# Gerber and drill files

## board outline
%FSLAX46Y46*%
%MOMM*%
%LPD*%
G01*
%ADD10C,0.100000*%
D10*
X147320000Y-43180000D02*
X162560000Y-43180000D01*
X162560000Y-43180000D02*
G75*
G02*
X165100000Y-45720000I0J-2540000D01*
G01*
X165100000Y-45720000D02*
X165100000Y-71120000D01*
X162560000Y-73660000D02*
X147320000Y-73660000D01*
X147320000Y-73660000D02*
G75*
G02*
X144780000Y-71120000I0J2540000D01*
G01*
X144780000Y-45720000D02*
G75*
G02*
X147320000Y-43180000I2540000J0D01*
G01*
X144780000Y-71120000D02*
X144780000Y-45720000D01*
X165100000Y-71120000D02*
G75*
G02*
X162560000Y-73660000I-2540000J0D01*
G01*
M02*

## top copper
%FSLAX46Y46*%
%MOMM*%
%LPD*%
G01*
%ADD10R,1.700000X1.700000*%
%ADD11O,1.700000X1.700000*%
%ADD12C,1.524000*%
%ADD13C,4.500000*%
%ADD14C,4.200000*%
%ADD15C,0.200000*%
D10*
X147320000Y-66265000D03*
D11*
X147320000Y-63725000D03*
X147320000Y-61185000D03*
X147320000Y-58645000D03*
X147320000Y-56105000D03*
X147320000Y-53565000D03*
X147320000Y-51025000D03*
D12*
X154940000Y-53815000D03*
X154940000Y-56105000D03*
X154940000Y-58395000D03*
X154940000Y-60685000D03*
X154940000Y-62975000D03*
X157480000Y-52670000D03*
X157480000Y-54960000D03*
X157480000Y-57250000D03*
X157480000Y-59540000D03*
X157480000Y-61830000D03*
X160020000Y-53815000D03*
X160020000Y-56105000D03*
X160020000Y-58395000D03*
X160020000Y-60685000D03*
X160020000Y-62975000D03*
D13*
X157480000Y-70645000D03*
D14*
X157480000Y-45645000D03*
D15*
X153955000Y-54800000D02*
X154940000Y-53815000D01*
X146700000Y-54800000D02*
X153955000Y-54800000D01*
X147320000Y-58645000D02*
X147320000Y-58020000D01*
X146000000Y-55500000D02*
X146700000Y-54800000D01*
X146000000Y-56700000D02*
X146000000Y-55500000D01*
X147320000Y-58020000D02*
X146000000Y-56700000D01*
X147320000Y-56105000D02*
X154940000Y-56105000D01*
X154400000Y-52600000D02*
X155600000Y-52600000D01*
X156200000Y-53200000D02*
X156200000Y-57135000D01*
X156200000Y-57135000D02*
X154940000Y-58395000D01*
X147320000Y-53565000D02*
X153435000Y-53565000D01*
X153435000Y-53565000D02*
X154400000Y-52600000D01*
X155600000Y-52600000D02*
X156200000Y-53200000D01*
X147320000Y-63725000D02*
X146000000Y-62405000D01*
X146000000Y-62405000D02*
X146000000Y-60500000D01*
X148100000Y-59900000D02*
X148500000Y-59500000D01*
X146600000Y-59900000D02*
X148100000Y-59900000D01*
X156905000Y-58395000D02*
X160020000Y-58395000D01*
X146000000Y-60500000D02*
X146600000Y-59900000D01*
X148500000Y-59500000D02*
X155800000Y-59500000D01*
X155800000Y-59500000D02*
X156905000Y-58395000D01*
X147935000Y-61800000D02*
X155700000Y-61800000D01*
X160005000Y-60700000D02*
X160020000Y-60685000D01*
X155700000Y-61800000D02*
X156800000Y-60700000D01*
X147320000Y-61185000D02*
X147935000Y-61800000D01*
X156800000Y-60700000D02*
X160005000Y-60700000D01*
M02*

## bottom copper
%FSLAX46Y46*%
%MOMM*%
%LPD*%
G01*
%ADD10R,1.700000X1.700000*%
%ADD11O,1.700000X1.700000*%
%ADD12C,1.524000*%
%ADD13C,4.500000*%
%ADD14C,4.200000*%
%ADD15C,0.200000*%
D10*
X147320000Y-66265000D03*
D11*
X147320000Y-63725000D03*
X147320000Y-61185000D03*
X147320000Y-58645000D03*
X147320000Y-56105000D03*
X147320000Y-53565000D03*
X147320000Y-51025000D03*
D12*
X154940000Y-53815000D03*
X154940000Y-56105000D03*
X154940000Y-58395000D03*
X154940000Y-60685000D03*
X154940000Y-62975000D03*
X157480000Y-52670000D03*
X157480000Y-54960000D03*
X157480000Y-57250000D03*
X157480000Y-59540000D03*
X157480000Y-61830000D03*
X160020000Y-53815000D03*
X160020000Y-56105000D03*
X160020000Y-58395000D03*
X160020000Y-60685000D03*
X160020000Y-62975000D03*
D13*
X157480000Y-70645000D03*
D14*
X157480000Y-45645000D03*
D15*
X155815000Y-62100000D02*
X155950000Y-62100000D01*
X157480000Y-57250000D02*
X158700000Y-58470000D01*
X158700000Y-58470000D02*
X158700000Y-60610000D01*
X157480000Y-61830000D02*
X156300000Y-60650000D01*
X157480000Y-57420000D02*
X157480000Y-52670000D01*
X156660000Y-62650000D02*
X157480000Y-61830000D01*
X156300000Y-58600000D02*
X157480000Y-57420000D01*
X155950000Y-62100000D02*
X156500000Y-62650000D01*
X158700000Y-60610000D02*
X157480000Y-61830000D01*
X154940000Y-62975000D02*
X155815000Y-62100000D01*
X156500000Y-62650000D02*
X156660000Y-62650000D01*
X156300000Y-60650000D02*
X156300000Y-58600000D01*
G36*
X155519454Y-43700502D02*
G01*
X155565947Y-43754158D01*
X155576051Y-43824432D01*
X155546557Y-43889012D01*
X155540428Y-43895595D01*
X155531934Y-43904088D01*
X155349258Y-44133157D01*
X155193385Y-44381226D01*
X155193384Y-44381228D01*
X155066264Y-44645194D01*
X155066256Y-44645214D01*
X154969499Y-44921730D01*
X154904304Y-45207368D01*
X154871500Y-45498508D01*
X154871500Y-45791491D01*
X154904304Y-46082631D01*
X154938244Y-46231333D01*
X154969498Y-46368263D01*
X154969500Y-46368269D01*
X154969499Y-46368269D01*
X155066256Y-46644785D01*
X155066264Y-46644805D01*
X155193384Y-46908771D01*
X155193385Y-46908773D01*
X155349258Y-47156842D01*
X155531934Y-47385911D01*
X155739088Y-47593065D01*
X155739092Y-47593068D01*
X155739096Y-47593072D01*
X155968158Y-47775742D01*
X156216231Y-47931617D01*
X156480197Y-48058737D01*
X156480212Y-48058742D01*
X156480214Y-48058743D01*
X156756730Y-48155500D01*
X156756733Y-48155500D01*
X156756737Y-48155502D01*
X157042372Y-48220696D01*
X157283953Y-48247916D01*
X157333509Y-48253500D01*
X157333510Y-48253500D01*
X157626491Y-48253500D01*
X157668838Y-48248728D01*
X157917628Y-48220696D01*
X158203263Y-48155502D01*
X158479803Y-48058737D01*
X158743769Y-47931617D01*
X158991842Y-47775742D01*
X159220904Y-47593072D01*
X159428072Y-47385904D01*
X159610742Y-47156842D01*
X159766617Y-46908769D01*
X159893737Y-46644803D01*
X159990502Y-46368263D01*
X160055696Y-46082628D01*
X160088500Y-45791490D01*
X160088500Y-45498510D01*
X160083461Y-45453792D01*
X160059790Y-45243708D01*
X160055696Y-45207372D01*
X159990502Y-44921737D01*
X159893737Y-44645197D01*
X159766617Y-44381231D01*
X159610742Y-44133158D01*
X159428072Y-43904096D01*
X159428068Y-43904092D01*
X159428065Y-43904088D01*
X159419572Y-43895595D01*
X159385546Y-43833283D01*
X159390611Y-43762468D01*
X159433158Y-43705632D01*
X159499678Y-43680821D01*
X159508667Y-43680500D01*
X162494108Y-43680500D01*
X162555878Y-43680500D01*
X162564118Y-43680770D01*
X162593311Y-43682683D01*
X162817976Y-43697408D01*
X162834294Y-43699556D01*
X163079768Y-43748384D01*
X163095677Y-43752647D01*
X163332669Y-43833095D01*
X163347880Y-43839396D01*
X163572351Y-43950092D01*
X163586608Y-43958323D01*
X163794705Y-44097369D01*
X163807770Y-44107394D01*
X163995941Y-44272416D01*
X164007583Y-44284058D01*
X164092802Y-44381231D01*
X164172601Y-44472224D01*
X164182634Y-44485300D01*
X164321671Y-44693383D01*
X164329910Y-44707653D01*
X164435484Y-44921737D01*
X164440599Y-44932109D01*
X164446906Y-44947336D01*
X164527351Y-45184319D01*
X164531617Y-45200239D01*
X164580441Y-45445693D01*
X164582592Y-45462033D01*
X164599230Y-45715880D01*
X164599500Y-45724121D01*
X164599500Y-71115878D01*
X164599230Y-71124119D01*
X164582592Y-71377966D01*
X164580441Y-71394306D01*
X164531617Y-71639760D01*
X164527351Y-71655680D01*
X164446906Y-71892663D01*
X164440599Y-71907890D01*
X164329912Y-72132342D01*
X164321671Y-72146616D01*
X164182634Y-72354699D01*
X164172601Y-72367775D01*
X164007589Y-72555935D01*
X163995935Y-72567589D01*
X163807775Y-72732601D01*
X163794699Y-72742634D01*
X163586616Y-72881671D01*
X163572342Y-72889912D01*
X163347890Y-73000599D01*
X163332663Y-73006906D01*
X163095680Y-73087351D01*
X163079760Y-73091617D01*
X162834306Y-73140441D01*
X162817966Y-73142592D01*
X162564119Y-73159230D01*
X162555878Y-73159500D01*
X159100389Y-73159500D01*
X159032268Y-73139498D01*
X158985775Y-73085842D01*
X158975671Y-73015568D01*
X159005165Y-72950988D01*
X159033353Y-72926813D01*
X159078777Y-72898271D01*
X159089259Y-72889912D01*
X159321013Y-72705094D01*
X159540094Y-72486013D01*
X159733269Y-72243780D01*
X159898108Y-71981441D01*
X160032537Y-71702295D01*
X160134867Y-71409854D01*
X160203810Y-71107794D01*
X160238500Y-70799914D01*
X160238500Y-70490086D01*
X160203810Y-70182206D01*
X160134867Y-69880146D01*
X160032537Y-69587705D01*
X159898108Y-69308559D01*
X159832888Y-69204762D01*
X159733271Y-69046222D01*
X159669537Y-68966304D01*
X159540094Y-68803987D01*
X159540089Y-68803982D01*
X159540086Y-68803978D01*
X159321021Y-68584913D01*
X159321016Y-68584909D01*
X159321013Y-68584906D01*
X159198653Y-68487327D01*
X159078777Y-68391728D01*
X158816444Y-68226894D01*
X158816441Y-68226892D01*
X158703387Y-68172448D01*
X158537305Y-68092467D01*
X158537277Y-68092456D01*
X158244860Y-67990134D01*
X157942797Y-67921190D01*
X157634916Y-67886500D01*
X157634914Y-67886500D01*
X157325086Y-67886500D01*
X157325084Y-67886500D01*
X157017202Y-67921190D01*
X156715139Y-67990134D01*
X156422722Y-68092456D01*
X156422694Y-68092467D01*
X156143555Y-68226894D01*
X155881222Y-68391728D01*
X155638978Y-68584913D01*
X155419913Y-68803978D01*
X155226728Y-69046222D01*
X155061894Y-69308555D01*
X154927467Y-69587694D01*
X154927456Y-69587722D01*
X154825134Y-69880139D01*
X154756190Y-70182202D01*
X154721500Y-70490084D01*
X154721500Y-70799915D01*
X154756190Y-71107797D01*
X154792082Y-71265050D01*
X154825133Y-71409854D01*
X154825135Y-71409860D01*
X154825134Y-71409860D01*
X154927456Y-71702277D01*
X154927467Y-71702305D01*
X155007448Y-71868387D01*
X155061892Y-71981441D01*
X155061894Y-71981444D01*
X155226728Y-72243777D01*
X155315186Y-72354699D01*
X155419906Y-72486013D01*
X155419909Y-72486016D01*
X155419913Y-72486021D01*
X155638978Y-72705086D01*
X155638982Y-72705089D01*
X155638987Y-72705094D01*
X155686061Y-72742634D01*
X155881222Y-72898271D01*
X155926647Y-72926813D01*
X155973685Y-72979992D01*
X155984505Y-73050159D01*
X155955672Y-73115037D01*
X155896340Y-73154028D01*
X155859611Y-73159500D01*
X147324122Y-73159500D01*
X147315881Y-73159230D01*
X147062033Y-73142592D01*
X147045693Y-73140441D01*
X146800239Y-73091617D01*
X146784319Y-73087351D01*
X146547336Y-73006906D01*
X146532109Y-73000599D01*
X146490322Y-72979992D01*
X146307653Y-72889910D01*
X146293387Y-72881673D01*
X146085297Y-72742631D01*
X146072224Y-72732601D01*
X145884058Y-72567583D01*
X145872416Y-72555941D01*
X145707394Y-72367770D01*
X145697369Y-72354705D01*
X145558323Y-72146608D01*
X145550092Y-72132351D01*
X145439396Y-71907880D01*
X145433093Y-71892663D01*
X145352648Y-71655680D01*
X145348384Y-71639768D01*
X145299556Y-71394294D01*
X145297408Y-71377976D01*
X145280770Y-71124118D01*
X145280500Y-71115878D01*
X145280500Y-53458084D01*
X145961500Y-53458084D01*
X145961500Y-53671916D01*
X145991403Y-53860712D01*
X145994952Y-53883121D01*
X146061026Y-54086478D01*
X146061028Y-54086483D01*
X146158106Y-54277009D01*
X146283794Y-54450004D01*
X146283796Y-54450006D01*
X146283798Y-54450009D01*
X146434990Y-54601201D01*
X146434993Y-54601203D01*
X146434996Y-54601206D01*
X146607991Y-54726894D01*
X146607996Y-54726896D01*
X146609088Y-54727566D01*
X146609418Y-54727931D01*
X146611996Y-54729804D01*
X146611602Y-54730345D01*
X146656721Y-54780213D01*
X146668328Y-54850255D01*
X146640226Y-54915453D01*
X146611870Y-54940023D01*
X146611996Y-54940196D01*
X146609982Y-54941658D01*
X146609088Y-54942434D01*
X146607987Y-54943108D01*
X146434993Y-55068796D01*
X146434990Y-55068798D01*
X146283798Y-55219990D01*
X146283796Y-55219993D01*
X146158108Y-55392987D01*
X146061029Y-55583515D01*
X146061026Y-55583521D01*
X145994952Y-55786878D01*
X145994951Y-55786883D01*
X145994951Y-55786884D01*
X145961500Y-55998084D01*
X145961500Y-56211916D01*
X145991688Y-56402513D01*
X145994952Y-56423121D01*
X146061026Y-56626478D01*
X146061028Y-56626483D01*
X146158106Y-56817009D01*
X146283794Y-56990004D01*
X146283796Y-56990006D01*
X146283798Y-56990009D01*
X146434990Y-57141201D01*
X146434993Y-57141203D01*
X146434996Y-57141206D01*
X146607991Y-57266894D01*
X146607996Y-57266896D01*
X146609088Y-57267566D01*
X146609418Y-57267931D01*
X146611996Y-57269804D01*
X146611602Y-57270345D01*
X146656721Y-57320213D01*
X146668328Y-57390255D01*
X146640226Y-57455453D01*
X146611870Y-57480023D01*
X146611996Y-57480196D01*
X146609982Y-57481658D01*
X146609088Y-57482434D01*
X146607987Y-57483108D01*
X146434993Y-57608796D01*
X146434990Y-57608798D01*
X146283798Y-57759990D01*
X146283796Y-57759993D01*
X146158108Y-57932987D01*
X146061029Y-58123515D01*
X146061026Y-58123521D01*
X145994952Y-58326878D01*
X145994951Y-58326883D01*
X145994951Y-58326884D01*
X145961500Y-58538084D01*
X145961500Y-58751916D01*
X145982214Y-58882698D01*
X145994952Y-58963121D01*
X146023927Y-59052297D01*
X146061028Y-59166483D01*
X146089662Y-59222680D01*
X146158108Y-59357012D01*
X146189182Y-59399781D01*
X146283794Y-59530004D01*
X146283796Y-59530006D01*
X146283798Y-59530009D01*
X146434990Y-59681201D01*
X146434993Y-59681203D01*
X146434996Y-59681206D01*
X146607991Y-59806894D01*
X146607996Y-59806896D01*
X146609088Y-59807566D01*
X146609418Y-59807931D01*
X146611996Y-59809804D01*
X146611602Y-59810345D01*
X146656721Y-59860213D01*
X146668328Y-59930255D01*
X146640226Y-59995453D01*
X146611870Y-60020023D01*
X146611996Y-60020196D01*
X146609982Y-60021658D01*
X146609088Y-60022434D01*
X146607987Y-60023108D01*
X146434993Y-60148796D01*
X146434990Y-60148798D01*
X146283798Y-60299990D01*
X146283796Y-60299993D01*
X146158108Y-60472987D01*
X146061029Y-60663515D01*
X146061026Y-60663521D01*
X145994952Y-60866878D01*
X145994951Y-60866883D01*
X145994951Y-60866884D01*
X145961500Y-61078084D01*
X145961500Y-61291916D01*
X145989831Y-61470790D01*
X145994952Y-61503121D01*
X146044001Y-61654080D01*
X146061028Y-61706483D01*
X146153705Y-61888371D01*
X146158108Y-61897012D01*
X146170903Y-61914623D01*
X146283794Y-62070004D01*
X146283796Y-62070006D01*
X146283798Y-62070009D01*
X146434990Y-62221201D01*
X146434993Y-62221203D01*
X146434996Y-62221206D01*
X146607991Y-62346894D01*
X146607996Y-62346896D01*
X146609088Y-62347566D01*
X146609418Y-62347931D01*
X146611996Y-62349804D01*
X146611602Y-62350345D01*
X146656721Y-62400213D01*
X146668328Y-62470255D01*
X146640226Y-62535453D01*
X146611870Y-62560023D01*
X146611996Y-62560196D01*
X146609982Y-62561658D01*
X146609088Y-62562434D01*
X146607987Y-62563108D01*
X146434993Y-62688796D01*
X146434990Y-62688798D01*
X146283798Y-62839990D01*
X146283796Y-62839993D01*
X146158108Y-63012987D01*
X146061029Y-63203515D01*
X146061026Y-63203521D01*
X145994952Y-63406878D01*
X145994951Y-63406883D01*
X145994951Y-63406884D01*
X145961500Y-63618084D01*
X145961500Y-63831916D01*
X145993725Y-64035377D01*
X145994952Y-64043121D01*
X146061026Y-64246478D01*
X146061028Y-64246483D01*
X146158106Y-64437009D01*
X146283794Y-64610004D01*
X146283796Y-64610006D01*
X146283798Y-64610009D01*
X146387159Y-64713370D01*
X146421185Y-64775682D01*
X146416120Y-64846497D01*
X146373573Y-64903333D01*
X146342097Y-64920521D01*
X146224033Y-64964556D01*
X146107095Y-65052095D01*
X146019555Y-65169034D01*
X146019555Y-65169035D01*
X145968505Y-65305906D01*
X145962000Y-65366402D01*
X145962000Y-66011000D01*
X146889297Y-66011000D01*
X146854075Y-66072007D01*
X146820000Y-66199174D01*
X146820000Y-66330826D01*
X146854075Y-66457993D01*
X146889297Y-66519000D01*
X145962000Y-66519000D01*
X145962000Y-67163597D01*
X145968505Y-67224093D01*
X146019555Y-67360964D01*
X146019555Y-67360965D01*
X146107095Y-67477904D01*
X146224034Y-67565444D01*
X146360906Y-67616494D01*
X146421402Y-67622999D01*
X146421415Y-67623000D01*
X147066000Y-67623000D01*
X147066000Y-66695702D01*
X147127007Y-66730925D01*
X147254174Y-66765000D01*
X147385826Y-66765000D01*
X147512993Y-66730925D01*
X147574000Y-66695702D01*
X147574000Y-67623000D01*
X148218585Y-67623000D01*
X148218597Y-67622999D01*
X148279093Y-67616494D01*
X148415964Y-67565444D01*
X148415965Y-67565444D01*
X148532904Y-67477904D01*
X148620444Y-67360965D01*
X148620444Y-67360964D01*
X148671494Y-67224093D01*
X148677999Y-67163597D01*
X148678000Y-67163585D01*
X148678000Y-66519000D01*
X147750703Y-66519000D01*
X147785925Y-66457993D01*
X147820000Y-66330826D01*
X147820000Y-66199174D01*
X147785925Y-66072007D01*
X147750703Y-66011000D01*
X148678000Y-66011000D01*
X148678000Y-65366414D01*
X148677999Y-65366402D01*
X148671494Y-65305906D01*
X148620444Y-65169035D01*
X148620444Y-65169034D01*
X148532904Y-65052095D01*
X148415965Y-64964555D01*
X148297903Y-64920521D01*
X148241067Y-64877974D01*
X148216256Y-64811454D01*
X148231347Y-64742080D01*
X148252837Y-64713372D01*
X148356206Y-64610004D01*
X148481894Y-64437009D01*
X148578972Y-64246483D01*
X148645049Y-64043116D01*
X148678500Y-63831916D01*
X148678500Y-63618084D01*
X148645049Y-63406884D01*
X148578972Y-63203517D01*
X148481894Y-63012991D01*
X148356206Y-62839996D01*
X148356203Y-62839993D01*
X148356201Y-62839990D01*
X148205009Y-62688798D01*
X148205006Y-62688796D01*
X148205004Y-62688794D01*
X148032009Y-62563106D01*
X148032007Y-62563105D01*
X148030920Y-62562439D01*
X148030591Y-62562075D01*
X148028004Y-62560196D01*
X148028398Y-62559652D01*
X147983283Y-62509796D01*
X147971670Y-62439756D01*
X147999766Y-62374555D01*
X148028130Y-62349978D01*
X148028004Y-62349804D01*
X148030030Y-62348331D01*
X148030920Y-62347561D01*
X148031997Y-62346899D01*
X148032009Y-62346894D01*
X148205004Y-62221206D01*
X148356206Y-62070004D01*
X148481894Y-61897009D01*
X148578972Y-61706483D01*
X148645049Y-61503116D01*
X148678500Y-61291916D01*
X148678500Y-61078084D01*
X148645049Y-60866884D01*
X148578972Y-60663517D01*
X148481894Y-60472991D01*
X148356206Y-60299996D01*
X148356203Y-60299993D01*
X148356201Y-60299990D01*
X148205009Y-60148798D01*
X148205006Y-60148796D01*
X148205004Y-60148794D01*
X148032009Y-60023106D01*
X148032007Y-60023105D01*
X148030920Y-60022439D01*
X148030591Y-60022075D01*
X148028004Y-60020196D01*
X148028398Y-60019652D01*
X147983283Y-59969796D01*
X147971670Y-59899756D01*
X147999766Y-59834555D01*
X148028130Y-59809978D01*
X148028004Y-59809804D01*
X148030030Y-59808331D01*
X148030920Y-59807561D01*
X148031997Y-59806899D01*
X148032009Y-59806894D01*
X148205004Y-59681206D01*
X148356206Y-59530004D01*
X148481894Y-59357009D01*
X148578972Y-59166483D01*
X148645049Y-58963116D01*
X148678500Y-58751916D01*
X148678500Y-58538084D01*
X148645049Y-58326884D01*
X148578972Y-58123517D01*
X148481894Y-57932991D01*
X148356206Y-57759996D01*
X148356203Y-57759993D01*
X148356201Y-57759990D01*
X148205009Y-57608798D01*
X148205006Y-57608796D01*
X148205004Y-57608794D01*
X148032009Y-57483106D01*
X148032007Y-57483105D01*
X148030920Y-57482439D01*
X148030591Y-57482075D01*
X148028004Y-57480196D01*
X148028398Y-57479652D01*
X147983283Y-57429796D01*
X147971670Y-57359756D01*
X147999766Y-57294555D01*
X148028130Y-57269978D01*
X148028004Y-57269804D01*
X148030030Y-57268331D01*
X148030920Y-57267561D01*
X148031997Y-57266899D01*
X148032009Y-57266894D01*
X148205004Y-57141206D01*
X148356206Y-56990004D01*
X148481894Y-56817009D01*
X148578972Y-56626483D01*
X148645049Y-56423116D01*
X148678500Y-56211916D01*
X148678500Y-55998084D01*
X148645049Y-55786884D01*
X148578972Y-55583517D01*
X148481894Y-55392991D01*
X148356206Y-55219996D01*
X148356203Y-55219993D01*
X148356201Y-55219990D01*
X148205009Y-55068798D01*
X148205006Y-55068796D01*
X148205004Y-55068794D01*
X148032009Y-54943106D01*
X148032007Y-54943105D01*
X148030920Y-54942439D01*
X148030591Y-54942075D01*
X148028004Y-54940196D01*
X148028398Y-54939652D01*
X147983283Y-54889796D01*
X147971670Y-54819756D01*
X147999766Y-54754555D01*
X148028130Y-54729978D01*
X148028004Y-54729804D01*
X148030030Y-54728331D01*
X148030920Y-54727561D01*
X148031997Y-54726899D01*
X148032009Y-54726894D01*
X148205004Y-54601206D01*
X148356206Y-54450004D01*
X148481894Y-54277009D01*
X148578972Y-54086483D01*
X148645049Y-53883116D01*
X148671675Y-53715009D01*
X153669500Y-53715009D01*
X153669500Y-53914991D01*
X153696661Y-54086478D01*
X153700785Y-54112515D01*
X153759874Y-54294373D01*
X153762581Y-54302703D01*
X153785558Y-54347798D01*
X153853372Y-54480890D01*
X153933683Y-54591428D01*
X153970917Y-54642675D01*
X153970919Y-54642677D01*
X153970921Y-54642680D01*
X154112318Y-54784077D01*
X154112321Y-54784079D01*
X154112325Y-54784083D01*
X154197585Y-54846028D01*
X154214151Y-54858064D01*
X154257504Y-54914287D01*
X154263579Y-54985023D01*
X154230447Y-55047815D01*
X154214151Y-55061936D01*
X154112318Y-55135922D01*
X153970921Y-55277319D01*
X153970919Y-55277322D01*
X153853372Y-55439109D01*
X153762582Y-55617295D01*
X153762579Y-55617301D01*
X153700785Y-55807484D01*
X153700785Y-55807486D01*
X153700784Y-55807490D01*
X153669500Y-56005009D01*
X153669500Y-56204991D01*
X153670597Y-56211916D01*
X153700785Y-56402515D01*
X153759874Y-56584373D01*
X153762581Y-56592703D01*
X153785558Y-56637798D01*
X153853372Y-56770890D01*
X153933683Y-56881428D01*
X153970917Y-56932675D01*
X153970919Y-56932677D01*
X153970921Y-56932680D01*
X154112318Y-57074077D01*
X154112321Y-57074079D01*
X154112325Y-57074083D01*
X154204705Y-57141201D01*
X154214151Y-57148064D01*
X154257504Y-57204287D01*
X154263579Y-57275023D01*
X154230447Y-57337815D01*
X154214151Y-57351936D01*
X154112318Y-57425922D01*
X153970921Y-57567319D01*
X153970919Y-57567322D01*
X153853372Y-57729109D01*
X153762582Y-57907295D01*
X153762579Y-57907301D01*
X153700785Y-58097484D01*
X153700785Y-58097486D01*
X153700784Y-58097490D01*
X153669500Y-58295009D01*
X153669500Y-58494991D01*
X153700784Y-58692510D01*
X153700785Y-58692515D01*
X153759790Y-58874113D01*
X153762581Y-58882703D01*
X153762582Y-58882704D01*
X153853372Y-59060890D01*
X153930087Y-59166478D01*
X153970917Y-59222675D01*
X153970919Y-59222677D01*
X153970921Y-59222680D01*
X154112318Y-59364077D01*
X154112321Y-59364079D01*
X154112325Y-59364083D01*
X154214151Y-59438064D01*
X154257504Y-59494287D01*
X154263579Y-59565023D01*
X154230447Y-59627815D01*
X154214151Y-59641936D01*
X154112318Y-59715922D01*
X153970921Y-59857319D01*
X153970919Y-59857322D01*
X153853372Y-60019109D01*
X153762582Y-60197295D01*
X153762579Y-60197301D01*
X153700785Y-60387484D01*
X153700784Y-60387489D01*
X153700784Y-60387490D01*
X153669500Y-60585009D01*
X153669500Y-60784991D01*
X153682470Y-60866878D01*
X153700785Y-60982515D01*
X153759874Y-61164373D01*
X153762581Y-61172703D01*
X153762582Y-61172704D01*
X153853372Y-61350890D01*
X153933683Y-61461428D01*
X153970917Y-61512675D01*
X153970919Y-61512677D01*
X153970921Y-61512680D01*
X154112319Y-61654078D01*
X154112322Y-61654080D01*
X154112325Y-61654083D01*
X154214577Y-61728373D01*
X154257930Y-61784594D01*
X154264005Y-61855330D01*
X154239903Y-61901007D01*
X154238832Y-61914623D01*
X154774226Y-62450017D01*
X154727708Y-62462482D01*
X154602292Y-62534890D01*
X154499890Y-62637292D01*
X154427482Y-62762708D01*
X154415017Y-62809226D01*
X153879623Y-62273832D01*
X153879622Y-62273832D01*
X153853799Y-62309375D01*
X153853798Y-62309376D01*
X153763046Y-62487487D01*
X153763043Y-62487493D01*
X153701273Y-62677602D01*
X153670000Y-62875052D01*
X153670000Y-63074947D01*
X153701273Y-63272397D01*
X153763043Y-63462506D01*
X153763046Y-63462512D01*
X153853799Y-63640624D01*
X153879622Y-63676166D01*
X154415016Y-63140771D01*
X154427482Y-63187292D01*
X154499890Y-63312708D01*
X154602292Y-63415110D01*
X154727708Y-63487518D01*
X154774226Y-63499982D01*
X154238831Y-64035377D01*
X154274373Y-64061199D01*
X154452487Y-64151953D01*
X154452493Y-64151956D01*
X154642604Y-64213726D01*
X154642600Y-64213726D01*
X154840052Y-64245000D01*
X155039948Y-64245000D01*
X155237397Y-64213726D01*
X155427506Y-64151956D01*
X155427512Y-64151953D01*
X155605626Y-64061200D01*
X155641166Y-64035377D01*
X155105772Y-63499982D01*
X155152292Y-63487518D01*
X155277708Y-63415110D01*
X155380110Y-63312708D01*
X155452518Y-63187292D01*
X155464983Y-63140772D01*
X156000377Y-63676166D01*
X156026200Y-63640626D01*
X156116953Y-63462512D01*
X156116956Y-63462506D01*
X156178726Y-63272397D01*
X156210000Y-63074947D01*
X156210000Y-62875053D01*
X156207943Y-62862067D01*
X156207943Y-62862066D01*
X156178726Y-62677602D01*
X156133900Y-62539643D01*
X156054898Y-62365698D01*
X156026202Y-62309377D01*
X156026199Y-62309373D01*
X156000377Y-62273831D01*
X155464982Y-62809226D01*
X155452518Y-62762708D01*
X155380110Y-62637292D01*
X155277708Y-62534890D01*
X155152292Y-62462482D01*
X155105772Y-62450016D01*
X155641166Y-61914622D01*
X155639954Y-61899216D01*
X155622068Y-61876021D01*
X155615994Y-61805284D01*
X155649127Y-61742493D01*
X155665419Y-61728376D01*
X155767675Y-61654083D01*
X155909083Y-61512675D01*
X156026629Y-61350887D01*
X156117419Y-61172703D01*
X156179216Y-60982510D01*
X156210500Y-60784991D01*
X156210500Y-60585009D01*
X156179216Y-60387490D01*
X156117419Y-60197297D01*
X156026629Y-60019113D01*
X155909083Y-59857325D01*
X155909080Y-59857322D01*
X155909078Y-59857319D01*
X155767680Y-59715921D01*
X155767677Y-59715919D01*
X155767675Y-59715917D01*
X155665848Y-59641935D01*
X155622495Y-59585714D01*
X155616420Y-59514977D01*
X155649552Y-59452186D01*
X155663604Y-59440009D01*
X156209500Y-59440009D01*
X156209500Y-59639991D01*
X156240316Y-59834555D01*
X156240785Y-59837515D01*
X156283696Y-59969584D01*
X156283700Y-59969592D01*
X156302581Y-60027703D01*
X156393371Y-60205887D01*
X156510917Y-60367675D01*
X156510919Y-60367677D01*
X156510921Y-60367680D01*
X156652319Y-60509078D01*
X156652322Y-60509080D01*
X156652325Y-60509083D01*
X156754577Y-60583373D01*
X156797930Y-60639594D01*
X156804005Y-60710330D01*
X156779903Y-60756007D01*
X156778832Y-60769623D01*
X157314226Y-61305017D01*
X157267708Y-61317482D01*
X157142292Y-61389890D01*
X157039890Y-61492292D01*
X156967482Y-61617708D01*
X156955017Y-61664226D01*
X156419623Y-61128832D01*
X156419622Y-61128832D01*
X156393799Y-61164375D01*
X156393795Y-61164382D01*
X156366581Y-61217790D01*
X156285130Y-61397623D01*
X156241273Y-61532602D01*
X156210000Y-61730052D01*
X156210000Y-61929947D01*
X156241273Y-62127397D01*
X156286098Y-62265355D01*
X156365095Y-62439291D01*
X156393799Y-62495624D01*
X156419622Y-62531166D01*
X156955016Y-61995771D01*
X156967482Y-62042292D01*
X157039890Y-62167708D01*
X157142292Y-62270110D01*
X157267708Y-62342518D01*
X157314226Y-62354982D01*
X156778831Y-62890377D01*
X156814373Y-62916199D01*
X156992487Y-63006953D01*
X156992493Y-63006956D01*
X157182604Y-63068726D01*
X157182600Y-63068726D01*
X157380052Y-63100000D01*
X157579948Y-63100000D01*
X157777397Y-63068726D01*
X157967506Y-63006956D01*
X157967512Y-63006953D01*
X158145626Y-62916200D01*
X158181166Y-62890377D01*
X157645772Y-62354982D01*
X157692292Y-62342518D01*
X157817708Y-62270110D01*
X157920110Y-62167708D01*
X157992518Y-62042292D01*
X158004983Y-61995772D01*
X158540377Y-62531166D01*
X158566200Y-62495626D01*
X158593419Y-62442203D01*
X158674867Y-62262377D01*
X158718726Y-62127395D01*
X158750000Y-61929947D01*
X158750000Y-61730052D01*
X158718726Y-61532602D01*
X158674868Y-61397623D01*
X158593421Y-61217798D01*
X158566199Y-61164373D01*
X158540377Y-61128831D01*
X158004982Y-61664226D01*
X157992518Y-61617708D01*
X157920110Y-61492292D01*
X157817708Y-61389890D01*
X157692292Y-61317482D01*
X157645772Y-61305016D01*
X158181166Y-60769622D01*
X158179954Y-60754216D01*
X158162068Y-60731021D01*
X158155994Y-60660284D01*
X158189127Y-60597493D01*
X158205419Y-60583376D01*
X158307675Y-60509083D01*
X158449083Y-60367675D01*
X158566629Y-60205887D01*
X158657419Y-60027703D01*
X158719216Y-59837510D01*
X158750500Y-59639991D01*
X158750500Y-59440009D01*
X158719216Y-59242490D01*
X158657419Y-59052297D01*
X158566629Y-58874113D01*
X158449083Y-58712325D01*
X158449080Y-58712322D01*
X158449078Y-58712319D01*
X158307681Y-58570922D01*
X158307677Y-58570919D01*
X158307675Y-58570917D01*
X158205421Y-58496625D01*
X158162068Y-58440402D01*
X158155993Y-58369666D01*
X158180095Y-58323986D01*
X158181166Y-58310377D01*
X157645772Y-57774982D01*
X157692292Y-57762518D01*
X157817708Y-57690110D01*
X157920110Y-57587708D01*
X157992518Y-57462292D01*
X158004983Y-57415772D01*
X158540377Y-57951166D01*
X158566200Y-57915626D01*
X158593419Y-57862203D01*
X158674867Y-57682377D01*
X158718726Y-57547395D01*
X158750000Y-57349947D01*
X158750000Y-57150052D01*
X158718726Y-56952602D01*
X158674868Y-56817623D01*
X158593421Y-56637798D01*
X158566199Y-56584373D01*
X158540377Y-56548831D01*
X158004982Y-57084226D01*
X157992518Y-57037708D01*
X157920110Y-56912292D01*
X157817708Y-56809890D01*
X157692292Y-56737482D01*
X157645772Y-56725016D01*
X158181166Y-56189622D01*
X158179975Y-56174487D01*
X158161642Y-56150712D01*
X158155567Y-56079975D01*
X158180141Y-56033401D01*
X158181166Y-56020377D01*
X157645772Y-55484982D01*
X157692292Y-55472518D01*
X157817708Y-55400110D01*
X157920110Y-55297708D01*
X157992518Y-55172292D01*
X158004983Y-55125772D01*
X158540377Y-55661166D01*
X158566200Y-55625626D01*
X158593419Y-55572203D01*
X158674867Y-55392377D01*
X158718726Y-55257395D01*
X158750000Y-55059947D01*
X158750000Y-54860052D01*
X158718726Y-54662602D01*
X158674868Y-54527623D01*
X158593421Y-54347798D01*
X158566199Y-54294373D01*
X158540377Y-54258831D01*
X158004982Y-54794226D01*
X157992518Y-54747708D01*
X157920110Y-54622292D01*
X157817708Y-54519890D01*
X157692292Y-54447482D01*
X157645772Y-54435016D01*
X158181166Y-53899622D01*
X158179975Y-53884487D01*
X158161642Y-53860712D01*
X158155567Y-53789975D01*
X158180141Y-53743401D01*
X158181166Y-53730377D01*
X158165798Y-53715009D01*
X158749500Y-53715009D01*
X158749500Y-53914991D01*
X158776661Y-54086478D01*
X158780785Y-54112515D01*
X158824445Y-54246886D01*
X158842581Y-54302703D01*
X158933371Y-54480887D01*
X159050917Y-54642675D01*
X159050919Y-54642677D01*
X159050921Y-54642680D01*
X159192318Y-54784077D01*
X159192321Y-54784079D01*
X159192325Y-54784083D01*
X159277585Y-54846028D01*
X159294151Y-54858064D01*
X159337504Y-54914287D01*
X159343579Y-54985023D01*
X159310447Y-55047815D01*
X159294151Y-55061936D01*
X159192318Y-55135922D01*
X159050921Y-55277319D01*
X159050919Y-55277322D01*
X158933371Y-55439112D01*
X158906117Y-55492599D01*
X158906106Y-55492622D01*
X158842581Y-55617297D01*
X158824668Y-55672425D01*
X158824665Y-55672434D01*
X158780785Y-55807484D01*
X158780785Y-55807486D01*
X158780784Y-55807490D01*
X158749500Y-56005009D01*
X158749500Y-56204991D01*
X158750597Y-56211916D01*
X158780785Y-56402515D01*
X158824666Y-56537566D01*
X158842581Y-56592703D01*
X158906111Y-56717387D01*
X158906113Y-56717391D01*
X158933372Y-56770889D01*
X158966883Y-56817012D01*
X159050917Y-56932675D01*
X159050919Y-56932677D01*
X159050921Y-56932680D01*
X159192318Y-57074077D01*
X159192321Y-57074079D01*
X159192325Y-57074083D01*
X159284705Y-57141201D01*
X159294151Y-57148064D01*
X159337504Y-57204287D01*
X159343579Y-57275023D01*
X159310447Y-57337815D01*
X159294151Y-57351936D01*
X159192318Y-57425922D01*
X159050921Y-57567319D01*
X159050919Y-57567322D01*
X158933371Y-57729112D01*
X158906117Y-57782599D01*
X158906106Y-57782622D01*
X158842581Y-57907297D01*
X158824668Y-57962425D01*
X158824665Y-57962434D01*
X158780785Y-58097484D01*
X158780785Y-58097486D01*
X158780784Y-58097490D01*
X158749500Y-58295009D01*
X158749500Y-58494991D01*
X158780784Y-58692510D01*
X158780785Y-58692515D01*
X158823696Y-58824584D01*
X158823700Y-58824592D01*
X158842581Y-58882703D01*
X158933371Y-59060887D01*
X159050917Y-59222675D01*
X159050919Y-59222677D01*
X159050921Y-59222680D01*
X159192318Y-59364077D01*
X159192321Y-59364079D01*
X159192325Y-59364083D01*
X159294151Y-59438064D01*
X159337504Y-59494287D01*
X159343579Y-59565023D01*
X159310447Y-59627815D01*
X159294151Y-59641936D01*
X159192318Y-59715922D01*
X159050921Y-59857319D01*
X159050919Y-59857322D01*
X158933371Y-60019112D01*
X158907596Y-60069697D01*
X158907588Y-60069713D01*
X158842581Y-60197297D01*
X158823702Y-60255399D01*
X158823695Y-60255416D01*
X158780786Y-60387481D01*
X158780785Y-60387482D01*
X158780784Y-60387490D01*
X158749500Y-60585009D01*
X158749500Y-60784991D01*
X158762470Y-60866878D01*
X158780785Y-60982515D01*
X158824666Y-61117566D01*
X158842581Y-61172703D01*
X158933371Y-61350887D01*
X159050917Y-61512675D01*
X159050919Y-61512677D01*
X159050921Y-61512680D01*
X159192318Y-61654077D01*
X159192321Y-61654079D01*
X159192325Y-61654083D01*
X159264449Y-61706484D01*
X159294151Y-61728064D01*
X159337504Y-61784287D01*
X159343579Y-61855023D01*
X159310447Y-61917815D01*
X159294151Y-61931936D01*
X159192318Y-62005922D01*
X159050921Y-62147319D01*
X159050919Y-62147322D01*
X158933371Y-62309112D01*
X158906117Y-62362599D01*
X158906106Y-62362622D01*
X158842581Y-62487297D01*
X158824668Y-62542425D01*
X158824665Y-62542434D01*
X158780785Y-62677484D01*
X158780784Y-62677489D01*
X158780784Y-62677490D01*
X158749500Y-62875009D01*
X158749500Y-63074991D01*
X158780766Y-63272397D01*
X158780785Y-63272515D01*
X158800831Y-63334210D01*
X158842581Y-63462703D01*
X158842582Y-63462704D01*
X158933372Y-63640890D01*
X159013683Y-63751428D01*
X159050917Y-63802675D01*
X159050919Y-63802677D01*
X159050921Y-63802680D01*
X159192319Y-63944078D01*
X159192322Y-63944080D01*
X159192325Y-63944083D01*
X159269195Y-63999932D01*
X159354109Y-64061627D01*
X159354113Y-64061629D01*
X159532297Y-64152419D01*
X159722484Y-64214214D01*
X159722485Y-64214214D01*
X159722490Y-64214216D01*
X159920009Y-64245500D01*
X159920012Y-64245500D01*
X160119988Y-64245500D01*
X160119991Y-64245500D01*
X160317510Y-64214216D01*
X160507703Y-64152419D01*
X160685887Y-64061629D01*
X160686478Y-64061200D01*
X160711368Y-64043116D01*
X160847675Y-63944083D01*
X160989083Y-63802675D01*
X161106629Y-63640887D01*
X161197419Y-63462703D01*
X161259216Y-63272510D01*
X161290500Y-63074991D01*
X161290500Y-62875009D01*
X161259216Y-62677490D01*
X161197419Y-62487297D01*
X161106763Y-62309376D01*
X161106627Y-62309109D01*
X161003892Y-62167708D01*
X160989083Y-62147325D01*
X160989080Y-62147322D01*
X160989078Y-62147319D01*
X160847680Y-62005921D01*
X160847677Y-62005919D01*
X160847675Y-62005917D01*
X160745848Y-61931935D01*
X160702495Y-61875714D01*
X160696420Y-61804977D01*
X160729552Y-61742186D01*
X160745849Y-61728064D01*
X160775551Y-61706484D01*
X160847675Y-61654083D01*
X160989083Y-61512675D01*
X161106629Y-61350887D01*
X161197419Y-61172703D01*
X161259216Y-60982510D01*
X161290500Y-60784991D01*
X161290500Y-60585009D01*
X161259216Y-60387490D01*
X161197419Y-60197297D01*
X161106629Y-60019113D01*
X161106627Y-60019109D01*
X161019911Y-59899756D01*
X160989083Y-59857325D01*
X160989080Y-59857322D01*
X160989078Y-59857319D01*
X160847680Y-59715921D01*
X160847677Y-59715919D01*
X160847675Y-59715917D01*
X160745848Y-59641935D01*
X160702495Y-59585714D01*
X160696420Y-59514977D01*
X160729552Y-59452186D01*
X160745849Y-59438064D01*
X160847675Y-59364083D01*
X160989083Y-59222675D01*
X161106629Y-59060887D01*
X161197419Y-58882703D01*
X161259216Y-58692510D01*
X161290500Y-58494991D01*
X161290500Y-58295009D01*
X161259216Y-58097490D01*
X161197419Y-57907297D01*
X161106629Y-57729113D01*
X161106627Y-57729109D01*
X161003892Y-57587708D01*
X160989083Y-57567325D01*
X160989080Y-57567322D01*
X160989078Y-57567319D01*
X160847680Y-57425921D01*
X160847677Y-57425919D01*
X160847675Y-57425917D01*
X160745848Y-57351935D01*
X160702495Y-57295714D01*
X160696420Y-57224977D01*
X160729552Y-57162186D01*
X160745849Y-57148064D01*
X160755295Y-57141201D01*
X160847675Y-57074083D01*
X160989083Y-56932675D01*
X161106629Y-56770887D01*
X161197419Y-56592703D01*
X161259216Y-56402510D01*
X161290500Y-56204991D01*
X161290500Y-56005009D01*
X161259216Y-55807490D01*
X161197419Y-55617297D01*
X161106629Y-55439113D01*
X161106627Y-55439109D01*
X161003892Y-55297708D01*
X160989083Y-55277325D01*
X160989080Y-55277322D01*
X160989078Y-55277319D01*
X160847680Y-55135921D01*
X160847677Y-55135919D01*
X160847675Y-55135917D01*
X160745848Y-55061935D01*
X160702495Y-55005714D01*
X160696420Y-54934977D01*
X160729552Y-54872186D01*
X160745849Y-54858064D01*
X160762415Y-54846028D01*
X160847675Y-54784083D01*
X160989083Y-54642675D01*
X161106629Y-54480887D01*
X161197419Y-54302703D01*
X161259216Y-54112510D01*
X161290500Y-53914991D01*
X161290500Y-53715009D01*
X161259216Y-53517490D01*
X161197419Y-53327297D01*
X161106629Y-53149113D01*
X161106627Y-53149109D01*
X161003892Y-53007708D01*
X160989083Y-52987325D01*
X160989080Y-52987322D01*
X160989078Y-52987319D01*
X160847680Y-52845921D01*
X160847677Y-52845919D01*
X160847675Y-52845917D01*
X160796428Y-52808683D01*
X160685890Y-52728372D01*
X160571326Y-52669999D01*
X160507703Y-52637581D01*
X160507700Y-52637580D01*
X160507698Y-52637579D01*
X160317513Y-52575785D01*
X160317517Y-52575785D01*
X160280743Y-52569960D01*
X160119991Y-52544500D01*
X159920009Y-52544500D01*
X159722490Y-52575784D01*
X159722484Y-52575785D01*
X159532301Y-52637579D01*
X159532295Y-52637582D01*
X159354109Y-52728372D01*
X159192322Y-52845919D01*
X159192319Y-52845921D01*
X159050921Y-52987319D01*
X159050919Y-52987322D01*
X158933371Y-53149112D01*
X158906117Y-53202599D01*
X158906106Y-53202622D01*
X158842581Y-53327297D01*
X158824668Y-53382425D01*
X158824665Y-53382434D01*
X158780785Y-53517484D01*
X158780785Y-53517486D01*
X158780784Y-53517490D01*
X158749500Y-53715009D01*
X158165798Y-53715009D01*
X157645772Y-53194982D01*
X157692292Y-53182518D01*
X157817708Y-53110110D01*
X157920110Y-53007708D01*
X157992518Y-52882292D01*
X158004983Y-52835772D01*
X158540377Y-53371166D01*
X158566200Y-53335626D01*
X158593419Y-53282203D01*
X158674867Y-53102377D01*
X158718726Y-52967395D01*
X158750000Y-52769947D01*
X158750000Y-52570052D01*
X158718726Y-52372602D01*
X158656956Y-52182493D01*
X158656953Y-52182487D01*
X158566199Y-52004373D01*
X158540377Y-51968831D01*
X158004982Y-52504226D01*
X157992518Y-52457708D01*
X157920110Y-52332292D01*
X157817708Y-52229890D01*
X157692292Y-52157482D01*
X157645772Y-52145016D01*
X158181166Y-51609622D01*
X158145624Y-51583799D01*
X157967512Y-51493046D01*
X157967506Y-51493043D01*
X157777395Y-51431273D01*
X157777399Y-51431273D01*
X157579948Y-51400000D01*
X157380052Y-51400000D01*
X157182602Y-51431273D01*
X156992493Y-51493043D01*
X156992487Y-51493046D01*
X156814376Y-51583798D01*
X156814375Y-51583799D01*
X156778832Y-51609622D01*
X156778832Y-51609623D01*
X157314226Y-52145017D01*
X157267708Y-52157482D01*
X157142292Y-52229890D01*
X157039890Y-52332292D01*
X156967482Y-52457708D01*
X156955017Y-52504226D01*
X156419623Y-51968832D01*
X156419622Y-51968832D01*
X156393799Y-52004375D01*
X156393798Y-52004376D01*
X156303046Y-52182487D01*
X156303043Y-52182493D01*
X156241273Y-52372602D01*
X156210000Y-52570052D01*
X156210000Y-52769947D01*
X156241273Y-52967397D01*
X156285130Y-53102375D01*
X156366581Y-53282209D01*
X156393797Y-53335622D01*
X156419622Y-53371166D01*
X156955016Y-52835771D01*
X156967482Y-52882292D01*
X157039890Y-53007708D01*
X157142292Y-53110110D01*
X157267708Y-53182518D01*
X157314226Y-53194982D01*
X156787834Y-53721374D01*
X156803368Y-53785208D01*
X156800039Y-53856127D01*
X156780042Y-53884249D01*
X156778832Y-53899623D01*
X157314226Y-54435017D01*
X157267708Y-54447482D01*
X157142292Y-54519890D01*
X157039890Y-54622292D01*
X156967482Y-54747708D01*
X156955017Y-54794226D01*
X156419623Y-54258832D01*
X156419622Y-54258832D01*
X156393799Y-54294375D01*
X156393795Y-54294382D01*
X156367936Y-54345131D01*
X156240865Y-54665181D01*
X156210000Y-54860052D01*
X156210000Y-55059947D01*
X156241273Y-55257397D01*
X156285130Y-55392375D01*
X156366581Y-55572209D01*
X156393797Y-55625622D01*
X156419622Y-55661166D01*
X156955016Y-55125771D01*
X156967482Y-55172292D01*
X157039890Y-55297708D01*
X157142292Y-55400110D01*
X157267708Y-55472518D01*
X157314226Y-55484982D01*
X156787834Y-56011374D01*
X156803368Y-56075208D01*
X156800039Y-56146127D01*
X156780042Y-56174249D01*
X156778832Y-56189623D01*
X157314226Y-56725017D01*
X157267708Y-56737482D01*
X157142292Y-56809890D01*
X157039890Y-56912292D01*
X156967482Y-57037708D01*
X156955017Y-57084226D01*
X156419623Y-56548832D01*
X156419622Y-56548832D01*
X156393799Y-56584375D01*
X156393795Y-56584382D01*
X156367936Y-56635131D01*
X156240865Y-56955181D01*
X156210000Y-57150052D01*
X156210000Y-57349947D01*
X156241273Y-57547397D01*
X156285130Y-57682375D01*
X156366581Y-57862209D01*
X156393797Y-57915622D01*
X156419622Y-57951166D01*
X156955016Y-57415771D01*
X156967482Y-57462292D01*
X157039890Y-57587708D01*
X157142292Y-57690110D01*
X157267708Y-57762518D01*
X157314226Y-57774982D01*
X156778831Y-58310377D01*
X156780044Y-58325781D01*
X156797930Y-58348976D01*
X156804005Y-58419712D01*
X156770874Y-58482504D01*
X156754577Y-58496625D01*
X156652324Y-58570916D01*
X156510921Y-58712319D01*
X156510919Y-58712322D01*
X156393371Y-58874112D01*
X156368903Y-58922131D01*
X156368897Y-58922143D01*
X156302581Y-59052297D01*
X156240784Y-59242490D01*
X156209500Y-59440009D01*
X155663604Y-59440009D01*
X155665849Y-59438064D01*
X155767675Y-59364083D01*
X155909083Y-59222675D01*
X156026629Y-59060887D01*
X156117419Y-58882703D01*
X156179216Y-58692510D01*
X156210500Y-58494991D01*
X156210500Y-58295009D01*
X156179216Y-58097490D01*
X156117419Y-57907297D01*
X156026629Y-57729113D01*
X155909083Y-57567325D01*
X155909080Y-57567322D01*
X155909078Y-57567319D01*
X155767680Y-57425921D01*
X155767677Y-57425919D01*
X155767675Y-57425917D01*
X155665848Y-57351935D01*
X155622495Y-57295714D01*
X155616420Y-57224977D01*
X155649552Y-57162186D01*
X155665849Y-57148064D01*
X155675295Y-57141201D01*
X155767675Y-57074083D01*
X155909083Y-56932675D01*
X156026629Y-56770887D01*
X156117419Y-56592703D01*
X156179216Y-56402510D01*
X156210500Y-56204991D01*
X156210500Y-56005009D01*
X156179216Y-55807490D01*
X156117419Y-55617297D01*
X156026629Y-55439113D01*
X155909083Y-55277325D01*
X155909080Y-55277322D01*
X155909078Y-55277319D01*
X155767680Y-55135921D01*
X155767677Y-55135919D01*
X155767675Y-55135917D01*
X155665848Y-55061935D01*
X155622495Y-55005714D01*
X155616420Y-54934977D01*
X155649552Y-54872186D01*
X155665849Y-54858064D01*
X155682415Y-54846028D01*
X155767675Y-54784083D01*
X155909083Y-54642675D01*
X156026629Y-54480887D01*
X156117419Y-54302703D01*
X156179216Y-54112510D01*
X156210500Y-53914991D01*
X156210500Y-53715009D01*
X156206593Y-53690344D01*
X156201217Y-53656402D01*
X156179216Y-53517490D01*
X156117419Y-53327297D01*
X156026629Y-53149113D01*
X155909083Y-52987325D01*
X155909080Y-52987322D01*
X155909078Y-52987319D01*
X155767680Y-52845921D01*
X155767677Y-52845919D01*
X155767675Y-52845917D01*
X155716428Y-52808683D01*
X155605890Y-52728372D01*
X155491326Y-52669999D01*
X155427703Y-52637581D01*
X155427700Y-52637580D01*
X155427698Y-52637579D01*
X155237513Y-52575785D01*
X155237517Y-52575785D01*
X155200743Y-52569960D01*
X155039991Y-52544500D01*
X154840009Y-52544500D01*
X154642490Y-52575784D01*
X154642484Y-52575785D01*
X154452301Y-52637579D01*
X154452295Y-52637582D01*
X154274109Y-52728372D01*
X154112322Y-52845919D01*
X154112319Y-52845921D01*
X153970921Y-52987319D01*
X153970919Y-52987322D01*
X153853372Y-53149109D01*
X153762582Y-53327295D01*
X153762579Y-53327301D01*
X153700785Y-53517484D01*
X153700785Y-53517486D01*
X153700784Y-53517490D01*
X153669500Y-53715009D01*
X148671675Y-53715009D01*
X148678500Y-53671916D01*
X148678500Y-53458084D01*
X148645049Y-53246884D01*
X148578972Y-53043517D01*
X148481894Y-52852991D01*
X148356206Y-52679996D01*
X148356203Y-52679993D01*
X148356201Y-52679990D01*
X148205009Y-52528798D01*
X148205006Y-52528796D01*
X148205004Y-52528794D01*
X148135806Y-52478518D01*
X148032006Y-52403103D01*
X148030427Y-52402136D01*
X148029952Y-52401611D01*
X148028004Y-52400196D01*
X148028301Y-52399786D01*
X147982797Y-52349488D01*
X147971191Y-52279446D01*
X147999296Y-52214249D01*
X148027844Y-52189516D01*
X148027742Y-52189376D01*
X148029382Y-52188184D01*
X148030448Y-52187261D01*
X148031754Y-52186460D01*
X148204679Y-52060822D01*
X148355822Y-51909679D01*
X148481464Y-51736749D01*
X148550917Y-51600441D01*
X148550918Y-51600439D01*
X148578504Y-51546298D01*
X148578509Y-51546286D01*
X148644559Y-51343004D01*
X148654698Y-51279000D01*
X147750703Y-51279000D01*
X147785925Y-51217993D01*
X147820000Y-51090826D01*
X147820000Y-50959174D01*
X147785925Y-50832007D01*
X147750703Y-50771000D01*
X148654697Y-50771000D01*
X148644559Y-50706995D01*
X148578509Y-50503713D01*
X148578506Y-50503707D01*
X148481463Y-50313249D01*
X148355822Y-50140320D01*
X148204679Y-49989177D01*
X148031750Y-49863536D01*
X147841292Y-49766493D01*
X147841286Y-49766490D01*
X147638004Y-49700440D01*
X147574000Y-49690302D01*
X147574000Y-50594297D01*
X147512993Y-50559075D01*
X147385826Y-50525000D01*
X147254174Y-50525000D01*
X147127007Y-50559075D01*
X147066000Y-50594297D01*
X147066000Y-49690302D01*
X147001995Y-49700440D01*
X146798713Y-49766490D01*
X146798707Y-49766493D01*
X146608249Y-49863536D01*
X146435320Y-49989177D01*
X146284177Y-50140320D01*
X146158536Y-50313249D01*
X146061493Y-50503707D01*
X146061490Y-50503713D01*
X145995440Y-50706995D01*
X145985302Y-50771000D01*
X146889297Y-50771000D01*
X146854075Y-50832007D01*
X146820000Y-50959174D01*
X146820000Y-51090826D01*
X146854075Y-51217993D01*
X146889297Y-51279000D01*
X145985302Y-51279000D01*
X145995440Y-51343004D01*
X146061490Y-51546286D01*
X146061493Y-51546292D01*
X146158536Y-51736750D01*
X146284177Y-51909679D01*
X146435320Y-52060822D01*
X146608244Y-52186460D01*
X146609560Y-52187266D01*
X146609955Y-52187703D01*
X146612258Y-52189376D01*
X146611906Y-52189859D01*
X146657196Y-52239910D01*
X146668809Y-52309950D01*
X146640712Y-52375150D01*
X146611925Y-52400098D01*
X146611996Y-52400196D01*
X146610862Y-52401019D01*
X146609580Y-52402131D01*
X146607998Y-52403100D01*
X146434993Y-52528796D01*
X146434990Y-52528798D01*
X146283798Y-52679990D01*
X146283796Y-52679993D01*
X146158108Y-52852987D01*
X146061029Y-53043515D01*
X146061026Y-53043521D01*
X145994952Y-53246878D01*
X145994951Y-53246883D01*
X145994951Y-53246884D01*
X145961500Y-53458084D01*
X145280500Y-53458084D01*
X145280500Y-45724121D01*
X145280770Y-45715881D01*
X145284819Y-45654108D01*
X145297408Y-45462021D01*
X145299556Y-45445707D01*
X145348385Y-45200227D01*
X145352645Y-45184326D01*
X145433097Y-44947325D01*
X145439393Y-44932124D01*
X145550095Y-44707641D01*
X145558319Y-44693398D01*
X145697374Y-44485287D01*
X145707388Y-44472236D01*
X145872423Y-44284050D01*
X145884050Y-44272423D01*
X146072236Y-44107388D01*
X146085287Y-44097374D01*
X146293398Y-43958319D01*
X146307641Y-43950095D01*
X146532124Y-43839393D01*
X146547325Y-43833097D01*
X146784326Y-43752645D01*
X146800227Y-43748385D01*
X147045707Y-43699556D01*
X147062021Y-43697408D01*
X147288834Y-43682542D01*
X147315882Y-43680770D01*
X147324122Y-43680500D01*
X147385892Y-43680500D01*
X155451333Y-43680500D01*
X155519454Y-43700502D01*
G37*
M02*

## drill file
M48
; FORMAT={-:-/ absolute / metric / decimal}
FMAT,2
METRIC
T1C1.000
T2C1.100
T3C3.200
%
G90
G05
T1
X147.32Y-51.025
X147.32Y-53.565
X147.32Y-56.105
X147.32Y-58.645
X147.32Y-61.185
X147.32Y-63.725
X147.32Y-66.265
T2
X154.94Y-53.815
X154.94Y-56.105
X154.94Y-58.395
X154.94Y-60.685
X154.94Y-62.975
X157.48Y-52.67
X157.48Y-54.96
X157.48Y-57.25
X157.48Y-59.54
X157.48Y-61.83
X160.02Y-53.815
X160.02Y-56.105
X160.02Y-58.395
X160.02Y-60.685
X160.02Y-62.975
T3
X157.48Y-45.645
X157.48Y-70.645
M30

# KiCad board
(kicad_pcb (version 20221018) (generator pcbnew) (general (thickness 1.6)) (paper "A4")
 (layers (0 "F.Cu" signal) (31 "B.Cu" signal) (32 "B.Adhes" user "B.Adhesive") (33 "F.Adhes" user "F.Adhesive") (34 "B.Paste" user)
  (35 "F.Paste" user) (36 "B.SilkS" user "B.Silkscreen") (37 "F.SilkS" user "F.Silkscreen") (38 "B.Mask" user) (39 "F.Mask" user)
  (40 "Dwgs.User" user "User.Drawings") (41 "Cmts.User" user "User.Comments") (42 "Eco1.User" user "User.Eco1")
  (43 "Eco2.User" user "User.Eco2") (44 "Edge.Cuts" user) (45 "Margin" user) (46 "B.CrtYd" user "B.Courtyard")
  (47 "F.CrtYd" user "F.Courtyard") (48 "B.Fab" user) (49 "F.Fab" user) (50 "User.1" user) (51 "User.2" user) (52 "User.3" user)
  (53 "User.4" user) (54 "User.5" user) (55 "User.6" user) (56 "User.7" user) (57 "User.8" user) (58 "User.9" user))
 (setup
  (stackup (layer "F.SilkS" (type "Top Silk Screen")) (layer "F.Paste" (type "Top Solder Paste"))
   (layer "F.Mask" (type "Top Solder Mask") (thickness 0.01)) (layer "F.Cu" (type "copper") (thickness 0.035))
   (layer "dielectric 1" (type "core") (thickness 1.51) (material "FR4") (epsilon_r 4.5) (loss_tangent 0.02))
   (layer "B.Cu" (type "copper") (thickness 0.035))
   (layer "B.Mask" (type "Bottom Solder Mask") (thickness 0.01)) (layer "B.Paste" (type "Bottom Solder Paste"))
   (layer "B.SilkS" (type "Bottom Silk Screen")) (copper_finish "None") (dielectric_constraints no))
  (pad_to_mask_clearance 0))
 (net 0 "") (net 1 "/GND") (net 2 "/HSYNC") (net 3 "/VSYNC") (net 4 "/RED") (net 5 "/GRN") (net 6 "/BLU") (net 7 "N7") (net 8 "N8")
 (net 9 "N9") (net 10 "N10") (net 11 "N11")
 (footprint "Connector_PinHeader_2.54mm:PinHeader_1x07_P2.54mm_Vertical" (layer "F.Cu") (at 147.32 66.265 180)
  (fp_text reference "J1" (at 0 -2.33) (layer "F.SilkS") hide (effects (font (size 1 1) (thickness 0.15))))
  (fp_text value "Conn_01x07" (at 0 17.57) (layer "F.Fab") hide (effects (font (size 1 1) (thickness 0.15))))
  (pad "1" thru_hole rect (at 0 0 180) (size 1.7 1.7) (drill 1) (layers "*.Cu" "*.Mask") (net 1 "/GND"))
  (pad "2" thru_hole oval (at 0 2.54 180) (size 1.7 1.7) (drill 1) (layers "*.Cu" "*.Mask") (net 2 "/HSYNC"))
  (pad "3" thru_hole oval (at 0 5.08 180) (size 1.7 1.7) (drill 1) (layers "*.Cu" "*.Mask") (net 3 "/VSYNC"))
  (pad "4" thru_hole oval (at 0 7.62 180) (size 1.7 1.7) (drill 1) (layers "*.Cu" "*.Mask") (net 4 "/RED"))
  (pad "5" thru_hole oval (at 0 10.16 180) (size 1.7 1.7) (drill 1) (layers "*.Cu" "*.Mask") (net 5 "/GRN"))
  (pad "6" thru_hole oval (at 0 12.7 180) (size 1.7 1.7) (drill 1) (layers "*.Cu" "*.Mask") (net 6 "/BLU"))
  (pad "7" thru_hole oval (at 0 15.24 180) (size 1.7 1.7) (drill 1) (layers "*.Cu" "*.Mask") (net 1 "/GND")))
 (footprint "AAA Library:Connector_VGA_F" (layer "F.Cu") (at 160.02 58.395 90)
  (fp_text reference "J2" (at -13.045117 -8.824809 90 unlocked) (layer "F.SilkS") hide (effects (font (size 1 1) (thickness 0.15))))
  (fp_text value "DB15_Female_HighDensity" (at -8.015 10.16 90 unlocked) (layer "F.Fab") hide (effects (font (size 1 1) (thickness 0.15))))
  (pad "1" thru_hole circle (at 4.58 -5.08 90) (size 1.524 1.524) (drill 1.1) (layers "*.Cu" "*.Mask") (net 4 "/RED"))
  (pad "2" thru_hole circle (at 2.29 -5.08 90) (size 1.524 1.524) (drill 1.1) (layers "*.Cu" "*.Mask") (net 5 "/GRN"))
  (pad "3" thru_hole circle (at 0 -5.08 90) (size 1.524 1.524) (drill 1.1) (layers "*.Cu" "*.Mask") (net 6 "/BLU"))
  (pad "4" thru_hole circle (at -2.29 -5.08 90) (size 1.524 1.524) (drill 1.1) (layers "*.Cu" "*.Mask") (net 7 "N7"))
  (pad "5" thru_hole circle (at -4.58 -5.08 90) (size 1.524 1.524) (drill 1.1) (layers "*.Cu" "*.Mask") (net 1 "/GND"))
  (pad "6" thru_hole circle (at 5.725 -2.54 90) (size 1.524 1.524) (drill 1.1) (layers "*.Cu" "*.Mask") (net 1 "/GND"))
  (pad "7" thru_hole circle (at 3.435 -2.54 90) (size 1.524 1.524) (drill 1.1) (layers "*.Cu" "*.Mask") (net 1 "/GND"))
  (pad "8" thru_hole circle (at 1.145 -2.54 90) (size 1.524 1.524) (drill 1.1) (layers "*.Cu" "*.Mask") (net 1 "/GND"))
  (pad "9" thru_hole circle (at -1.145 -2.54 90) (size 1.524 1.524) (drill 1.1) (layers "*.Cu" "*.Mask") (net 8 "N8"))
  (pad "10" thru_hole circle (at -3.435 -2.54 90) (size 1.524 1.524) (drill 1.1) (layers "*.Cu" "*.Mask") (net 1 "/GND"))
  (pad "11" thru_hole circle (at 4.58 0 90) (size 1.524 1.524) (drill 1.1) (layers "*.Cu" "*.Mask") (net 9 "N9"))
  (pad "12" thru_hole circle (at 2.29 0 90) (size 1.524 1.524) (drill 1.1) (layers "*.Cu" "*.Mask") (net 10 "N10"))
  (pad "13" thru_hole circle (at 0 0 90) (size 1.524 1.524) (drill 1.1) (layers "*.Cu" "*.Mask") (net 2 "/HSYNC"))
  (pad "14" thru_hole circle (at -2.29 0 90) (size 1.524 1.524) (drill 1.1) (layers "*.Cu" "*.Mask") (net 3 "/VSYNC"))
  (pad "15" thru_hole circle (at -4.58 0 90) (size 1.524 1.524) (drill 1.1) (layers "*.Cu" "*.Mask") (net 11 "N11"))
  (pad "16" thru_hole circle (at -12.25 -2.54 90) (size 4.5 4.5) (drill 3.2) (layers "*.Cu" "*.Mask"))
  (pad "17" thru_hole circle (at 12.75 -2.54 90) (size 4.2 4.2) (drill 3.2) (layers "*.Cu" "*.Mask")))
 (gr_line (start 147.32 43.18) (end 162.56 43.18) (stroke (width 0.1) (type solid)) (layer "Edge.Cuts"))
 (gr_arc (start 162.56 43.18) (mid 164.356051 43.923949) (end 165.1 45.72) (stroke (width 0.1) (type solid)) (layer "Edge.Cuts"))
 (gr_line (start 165.1 45.72) (end 165.1 71.12) (stroke (width 0.1) (type solid)) (layer "Edge.Cuts"))
 (gr_line (start 162.56 73.66) (end 147.32 73.66) (stroke (width 0.1) (type solid)) (layer "Edge.Cuts"))
 (gr_arc (start 147.32 73.66) (mid 145.523949 72.916051) (end 144.78 71.12) (stroke (width 0.1) (type solid)) (layer "Edge.Cuts"))
 (gr_arc (start 144.78 45.72) (mid 145.523949 43.923949) (end 147.32 43.18) (stroke (width 0.1) (type solid)) (layer "Edge.Cuts"))
 (gr_line (start 144.78 71.12) (end 144.78 45.72) (stroke (width 0.1) (type solid)) (layer "Edge.Cuts"))
 (gr_arc (start 165.1 71.12) (mid 164.356051 72.916051) (end 162.56 73.66) (stroke (width 0.1) (type solid)) (layer "Edge.Cuts"))
 (segment (start 153.955 54.8) (end 154.94 53.815) (width 0.2) (layer "F.Cu") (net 4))
 (segment (start 146.7 54.8) (end 153.955 54.8) (width 0.2) (layer "F.Cu") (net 4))
 (segment (start 147.32 58.645) (end 147.32 58.02) (width 0.2) (layer "F.Cu") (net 4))
 (segment (start 146 55.5) (end 146.7 54.8) (width 0.2) (layer "F.Cu") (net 4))
 (segment (start 146 56.7) (end 146 55.5) (width 0.2) (layer "F.Cu") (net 4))
 (segment (start 147.32 58.02) (end 146 56.7) (width 0.2) (layer "F.Cu") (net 4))
 (segment (start 147.32 56.105) (end 154.94 56.105) (width 0.2) (layer "F.Cu") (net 5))
 (segment (start 154.4 52.6) (end 155.6 52.6) (width 0.2) (layer "F.Cu") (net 6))
 (segment (start 156.2 53.2) (end 156.2 57.135) (width 0.2) (layer "F.Cu") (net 6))
 (segment (start 156.2 57.135) (end 154.94 58.395) (width 0.2) (layer "F.Cu") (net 6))
 (segment (start 147.32 53.565) (end 153.435 53.565) (width 0.2) (layer "F.Cu") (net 6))
 (segment (start 153.435 53.565) (end 154.4 52.6) (width 0.2) (layer "F.Cu") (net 6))
 (segment (start 155.6 52.6) (end 156.2 53.2) (width 0.2) (layer "F.Cu") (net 6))
 (segment (start 155.815 62.1) (end 155.95 62.1) (width 0.2) (layer "B.Cu") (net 1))
 (segment (start 157.48 57.25) (end 158.7 58.47) (width 0.2) (layer "B.Cu") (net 1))
 (segment (start 158.7 58.47) (end 158.7 60.61) (width 0.2) (layer "B.Cu") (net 1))
 (segment (start 157.48 61.83) (end 156.3 60.65) (width 0.2) (layer "B.Cu") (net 1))
 (segment (start 157.48 57.42) (end 157.48 52.67) (width 0.2) (layer "B.Cu") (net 1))
 (segment (start 156.66 62.65) (end 157.48 61.83) (width 0.2) (layer "B.Cu") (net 1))
 (segment (start 156.3 58.6) (end 157.48 57.42) (width 0.2) (layer "B.Cu") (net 1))
 (segment (start 155.95 62.1) (end 156.5 62.65) (width 0.2) (layer "B.Cu") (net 1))
 (segment (start 158.7 60.61) (end 157.48 61.83) (width 0.2) (layer "B.Cu") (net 1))
 (segment (start 154.94 62.975) (end 155.815 62.1) (width 0.2) (layer "B.Cu") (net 1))
 (segment (start 156.5 62.65) (end 156.66 62.65) (width 0.2) (layer "B.Cu") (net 1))
 (segment (start 156.3 60.65) (end 156.3 58.6) (width 0.2) (layer "B.Cu") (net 1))
 (segment (start 147.32 63.725) (end 146 62.405) (width 0.2) (layer "F.Cu") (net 2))
 (segment (start 146 62.405) (end 146 60.5) (width 0.2) (layer "F.Cu") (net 2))
 (segment (start 148.1 59.9) (end 148.5 59.5) (width 0.2) (layer "F.Cu") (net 2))
 (segment (start 146.6 59.9) (end 148.1 59.9) (width 0.2) (layer "F.Cu") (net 2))
 (segment (start 156.905 58.395) (end 160.02 58.395) (width 0.2) (layer "F.Cu") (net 2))
 (segment (start 146 60.5) (end 146.6 59.9) (width 0.2) (layer "F.Cu") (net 2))
 (segment (start 148.5 59.5) (end 155.8 59.5) (width 0.2) (layer "F.Cu") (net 2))
 (segment (start 155.8 59.5) (end 156.905 58.395) (width 0.2) (layer "F.Cu") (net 2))
 (segment (start 147.935 61.8) (end 155.7 61.8) (width 0.2) (layer "F.Cu") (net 3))
 (segment (start 160.005 60.7) (end 160.02 60.685) (width 0.2) (layer "F.Cu") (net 3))
 (segment (start 155.7 61.8) (end 156.8 60.7) (width 0.2) (layer "F.Cu") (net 3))
 (segment (start 147.32 61.185) (end 147.935 61.8) (width 0.2) (layer "F.Cu") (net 3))
 (segment (start 156.8 60.7) (end 160.005 60.7) (width 0.2) (layer "F.Cu") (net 3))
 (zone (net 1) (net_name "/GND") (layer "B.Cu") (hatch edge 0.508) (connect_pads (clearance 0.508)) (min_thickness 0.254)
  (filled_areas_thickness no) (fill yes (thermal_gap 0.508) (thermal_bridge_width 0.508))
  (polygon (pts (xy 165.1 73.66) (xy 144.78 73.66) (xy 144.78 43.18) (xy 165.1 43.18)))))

